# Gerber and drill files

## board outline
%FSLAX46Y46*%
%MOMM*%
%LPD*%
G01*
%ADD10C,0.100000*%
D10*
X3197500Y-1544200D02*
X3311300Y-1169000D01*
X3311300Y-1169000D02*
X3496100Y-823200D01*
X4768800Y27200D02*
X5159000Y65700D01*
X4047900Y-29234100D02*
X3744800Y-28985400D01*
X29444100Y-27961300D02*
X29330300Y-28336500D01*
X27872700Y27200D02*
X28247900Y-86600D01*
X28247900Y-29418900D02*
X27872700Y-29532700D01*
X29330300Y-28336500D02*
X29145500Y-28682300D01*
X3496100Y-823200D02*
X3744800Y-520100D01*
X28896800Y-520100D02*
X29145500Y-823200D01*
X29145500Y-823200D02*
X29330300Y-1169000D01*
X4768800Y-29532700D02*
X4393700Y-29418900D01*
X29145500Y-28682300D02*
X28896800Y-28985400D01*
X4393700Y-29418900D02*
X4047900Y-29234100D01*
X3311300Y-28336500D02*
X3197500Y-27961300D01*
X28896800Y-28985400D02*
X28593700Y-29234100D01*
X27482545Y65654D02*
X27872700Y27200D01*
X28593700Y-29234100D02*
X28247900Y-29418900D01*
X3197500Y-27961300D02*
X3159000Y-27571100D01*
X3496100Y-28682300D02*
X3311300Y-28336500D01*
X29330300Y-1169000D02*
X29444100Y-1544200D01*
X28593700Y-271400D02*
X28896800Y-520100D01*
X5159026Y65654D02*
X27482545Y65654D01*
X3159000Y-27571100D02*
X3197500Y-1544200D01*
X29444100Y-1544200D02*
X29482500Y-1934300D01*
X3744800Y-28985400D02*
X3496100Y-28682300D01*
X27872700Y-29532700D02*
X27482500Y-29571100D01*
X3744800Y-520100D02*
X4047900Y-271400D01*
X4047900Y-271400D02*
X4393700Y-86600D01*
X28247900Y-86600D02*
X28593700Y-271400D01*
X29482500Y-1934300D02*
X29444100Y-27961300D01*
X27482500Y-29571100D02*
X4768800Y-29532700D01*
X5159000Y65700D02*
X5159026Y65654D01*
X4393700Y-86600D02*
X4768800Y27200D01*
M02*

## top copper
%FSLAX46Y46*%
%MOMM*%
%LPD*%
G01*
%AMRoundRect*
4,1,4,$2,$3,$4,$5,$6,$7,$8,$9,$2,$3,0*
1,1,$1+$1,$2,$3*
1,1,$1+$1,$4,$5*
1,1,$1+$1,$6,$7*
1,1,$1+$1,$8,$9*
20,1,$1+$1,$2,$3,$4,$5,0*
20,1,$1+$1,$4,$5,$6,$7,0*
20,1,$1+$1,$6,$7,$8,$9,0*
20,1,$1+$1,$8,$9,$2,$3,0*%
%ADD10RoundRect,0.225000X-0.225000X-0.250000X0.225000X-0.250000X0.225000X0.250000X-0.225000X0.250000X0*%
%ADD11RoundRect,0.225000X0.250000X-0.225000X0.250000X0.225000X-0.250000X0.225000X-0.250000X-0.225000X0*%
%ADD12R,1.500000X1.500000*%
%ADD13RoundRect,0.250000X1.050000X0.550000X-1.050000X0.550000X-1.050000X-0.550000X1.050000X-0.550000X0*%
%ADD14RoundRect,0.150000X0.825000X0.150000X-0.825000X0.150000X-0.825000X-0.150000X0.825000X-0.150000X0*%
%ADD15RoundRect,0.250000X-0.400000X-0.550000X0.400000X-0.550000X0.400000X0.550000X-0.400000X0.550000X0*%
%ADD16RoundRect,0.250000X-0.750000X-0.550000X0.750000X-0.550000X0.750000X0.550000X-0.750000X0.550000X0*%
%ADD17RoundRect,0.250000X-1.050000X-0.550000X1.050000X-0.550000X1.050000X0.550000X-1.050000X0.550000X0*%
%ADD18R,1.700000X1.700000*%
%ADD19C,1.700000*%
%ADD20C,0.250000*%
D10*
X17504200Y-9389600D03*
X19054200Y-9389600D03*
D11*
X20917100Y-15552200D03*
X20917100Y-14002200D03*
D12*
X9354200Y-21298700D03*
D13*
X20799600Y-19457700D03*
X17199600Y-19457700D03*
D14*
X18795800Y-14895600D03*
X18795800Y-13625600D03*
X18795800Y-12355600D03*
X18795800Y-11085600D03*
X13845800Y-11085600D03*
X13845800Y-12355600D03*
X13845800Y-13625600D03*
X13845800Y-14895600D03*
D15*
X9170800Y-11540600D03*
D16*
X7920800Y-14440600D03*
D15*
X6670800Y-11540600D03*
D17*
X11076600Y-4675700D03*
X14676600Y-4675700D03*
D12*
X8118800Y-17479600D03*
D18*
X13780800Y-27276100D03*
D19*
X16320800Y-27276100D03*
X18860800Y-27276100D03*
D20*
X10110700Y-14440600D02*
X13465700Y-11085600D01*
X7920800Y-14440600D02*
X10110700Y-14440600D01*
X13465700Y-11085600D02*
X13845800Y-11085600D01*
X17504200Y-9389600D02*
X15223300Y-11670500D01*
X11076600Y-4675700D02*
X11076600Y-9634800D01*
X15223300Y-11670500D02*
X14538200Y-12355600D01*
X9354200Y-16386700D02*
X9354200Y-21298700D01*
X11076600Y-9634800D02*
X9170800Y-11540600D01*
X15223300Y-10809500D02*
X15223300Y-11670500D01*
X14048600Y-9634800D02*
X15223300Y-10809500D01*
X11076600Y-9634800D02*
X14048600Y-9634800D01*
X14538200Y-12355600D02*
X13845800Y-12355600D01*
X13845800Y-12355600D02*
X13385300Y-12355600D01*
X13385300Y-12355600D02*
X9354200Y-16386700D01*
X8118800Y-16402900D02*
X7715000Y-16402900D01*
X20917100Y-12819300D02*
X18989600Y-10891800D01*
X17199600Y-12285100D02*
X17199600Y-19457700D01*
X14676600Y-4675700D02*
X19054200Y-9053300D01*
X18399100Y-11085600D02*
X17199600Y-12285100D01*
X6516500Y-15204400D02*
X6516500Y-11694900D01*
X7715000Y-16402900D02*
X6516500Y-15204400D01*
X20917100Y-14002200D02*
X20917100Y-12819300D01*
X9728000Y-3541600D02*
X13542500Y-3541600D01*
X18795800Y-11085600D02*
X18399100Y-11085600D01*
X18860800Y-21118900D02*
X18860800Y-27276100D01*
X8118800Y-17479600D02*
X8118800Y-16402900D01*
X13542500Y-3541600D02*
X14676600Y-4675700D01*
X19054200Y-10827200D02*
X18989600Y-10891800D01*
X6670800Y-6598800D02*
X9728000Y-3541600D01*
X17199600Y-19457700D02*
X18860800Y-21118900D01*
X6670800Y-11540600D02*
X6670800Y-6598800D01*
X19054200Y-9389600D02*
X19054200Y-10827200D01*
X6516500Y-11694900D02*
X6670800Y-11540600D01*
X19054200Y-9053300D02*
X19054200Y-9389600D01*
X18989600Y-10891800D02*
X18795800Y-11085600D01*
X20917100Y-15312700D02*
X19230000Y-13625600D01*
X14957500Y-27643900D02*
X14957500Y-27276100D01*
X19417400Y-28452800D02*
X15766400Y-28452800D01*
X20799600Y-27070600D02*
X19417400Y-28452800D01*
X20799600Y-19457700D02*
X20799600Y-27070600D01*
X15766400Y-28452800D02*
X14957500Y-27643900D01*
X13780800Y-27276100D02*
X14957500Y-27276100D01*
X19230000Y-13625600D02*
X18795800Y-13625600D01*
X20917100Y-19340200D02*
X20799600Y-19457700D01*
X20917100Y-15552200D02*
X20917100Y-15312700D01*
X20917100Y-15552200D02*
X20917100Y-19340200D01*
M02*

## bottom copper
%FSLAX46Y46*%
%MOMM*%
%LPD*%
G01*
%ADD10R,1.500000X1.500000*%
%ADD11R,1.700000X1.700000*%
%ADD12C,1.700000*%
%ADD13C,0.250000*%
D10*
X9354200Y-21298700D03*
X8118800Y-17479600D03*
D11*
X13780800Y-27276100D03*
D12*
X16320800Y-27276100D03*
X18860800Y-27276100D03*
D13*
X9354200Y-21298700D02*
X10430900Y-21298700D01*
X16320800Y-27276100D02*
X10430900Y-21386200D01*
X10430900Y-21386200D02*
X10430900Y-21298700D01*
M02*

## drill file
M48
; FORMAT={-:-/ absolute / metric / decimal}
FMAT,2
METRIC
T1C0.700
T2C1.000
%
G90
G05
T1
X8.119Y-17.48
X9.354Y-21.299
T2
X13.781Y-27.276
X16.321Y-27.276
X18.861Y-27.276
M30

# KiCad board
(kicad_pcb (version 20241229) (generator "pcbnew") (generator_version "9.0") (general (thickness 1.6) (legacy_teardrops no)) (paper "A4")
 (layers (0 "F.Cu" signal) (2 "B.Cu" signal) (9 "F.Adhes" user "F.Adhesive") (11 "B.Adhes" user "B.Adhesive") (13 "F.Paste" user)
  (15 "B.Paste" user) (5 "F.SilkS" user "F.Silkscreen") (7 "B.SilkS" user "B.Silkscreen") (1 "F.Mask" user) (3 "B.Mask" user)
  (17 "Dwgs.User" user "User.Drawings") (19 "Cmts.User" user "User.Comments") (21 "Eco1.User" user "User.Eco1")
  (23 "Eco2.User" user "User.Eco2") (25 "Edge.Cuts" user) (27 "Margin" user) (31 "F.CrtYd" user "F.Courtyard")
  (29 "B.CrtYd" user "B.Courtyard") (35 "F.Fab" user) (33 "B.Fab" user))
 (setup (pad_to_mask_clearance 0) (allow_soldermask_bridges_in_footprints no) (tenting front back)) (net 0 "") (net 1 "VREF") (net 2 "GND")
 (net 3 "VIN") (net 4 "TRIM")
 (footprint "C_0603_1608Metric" (layer "F.Cu") (at 18.2792 9.3896)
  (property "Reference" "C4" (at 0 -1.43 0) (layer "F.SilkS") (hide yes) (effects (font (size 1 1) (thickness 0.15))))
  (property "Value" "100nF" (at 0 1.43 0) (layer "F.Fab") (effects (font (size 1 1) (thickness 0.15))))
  (pad "1" smd roundrect (at -0.775 0) (size 0.9 0.95) (layers "F.Cu" "F.Mask" "F.Paste") (roundrect_rratio 0.25) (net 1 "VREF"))
  (pad "2" smd roundrect (at 0.775 0) (size 0.9 0.95) (layers "F.Cu" "F.Mask" "F.Paste") (roundrect_rratio 0.25) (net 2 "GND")))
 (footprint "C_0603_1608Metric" (layer "F.Cu") (at 20.9171 14.7772 90)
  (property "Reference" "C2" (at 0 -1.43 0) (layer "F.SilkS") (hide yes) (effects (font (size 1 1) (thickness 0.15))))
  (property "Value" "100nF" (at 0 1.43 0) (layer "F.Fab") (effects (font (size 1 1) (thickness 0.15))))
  (pad "1" smd roundrect (at -0.775 0 90) (size 0.9 0.95) (layers "F.Cu" "F.Mask" "F.Paste") (roundrect_rratio 0.25) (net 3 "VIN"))
  (pad "2" smd roundrect (at 0.775 0 90) (size 0.9 0.95) (layers "F.Cu" "F.Mask" "F.Paste") (roundrect_rratio 0.25) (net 2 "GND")))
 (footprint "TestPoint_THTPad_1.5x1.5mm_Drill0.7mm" (layer "F.Cu") (at 9.3542 21.2987)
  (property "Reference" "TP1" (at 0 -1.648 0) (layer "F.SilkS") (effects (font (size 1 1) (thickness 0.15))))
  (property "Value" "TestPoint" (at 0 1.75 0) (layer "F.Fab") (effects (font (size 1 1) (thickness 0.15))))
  (pad "1" thru_hole rect (at 0 0) (size 1.5 1.5) (drill 0.7) (layers "*.Cu" "*.Mask") (remove_unused_layers no) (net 1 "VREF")))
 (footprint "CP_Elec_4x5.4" (layer "F.Cu") (at 18.9996 19.4577 180)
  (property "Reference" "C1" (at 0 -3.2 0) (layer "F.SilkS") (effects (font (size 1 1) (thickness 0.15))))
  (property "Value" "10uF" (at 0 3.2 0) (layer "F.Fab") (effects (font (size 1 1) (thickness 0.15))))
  (pad "1" smd roundrect (at -1.8 0 180) (size 2.6 1.6) (layers "F.Cu" "F.Mask" "F.Paste") (roundrect_rratio 0.15625) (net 3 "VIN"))
  (pad "2" smd roundrect (at 1.8 0 180) (size 2.6 1.6) (layers "F.Cu" "F.Mask" "F.Paste") (roundrect_rratio 0.15625) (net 2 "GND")))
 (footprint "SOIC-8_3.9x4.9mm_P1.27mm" (layer "F.Cu") (at 16.3208 12.9906 180)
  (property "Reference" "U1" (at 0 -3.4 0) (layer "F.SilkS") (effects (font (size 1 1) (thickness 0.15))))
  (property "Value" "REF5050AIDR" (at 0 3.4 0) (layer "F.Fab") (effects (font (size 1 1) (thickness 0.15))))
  (pad "1" smd roundrect (at -2.475 -1.905 180) (size 1.95 0.6) (layers "F.Cu" "F.Mask" "F.Paste") (roundrect_rratio 0.25))
  (pad "2" smd roundrect (at -2.475 -0.635 180) (size 1.95 0.6) (layers "F.Cu" "F.Mask" "F.Paste") (roundrect_rratio 0.25) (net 3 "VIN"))
  (pad "3" smd roundrect (at -2.475 0.635 180) (size 1.95 0.6) (layers "F.Cu" "F.Mask" "F.Paste") (roundrect_rratio 0.25))
  (pad "4" smd roundrect (at -2.475 1.905 180) (size 1.95 0.6) (layers "F.Cu" "F.Mask" "F.Paste") (roundrect_rratio 0.25) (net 2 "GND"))
  (pad "5" smd roundrect (at 2.475 1.905 180) (size 1.95 0.6) (layers "F.Cu" "F.Mask" "F.Paste") (roundrect_rratio 0.25) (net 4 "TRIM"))
  (pad "6" smd roundrect (at 2.475 0.635 180) (size 1.95 0.6) (layers "F.Cu" "F.Mask" "F.Paste") (roundrect_rratio 0.25) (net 1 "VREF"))
  (pad "7" smd roundrect (at 2.475 -0.635 180) (size 1.95 0.6) (layers "F.Cu" "F.Mask" "F.Paste") (roundrect_rratio 0.25))
  (pad "8" smd roundrect (at 2.475 -1.905 180) (size 1.95 0.6) (layers "F.Cu" "F.Mask" "F.Paste") (roundrect_rratio 0.25)))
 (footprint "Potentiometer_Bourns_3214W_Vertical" (layer "F.Cu") (at 7.9208 12.9906)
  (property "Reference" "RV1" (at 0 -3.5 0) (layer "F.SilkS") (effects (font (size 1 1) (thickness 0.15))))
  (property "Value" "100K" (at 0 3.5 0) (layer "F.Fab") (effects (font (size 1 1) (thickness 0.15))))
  (pad "1" smd roundrect (at 1.25 -1.45) (size 1.3 1.6) (layers "F.Cu" "F.Mask" "F.Paste") (roundrect_rratio 0.192308) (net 1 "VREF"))
  (pad "2" smd roundrect (at 0 1.45) (size 2 1.6) (layers "F.Cu" "F.Mask" "F.Paste") (roundrect_rratio 0.15625) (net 4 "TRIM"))
  (pad "3" smd roundrect (at -1.25 -1.45) (size 1.3 1.6) (layers "F.Cu" "F.Mask" "F.Paste") (roundrect_rratio 0.192308) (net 2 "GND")))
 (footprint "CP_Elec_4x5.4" (layer "F.Cu") (at 12.8766 4.6757)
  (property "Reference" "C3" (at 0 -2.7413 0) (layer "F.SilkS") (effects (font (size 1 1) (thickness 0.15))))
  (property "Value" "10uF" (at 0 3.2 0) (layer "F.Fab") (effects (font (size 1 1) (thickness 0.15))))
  (pad "1" smd roundrect (at -1.8 0) (size 2.6 1.6) (layers "F.Cu" "F.Mask" "F.Paste") (roundrect_rratio 0.15625) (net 1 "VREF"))
  (pad "2" smd roundrect (at 1.8 0) (size 2.6 1.6) (layers "F.Cu" "F.Mask" "F.Paste") (roundrect_rratio 0.15625) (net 2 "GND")))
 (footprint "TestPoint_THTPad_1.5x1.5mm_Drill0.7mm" (layer "F.Cu") (at 8.1188 17.4796)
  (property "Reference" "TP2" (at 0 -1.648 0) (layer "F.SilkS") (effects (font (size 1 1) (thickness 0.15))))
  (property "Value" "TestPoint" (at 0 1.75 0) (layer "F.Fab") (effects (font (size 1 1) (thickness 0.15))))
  (pad "1" thru_hole rect (at 0 0) (size 1.5 1.5) (drill 0.7) (layers "*.Cu" "*.Mask") (remove_unused_layers no) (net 2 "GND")))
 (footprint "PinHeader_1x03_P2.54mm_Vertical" (layer "F.Cu") (at 13.7808 27.2761 90)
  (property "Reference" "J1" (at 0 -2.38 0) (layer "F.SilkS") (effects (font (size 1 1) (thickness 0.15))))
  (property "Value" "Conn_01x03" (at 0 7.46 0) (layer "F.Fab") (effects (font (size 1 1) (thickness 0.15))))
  (pad "1" thru_hole rect (at 0 0 90) (size 1.7 1.7) (drill 1) (layers "*.Cu" "*.Mask") (remove_unused_layers no) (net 3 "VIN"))
  (pad "2" thru_hole circle (at 0 2.54 90) (size 1.7 1.7) (drill 1) (layers "*.Cu" "*.Mask") (remove_unused_layers no) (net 1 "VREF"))
  (pad "3" thru_hole circle (at 0 5.08 90) (size 1.7 1.7) (drill 1) (layers "*.Cu" "*.Mask") (remove_unused_layers no) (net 2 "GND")))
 (gr_line (start 3.1975 1.5442) (end 3.3113 1.169) (stroke (width 0.1) (type solid)) (layer "Edge.Cuts"))
 (gr_line (start 3.3113 1.169) (end 3.4961 0.8232) (stroke (width 0.1) (type solid)) (layer "Edge.Cuts"))
 (gr_line (start 4.7688 -0.0272) (end 5.159 -0.0657) (stroke (width 0.1) (type solid)) (layer "Edge.Cuts"))
 (gr_line (start 4.0479 29.2341) (end 3.7448 28.9854) (stroke (width 0.1) (type solid)) (layer "Edge.Cuts"))
 (gr_line (start 29.4441 27.9613) (end 29.3303 28.3365) (stroke (width 0.1) (type solid)) (layer "Edge.Cuts"))
 (gr_line (start 27.8727 -0.0272) (end 28.2479 0.0866) (stroke (width 0.1) (type solid)) (layer "Edge.Cuts"))
 (gr_line (start 28.2479 29.4189) (end 27.8727 29.5327) (stroke (width 0.1) (type solid)) (layer "Edge.Cuts"))
 (gr_line (start 29.3303 28.3365) (end 29.1455 28.6823) (stroke (width 0.1) (type solid)) (layer "Edge.Cuts"))
 (gr_line (start 3.4961 0.8232) (end 3.7448 0.5201) (stroke (width 0.1) (type solid)) (layer "Edge.Cuts"))
 (gr_line (start 28.8968 0.5201) (end 29.1455 0.8232) (stroke (width 0.1) (type solid)) (layer "Edge.Cuts"))
 (gr_line (start 29.1455 0.8232) (end 29.3303 1.169) (stroke (width 0.1) (type solid)) (layer "Edge.Cuts"))
 (gr_line (start 4.7688 29.5327) (end 4.3937 29.4189) (stroke (width 0.1) (type solid)) (layer "Edge.Cuts"))
 (gr_line (start 29.1455 28.6823) (end 28.8968 28.9854) (stroke (width 0.1) (type solid)) (layer "Edge.Cuts"))
 (gr_line (start 4.3937 29.4189) (end 4.0479 29.2341) (stroke (width 0.1) (type solid)) (layer "Edge.Cuts"))
 (gr_line (start 3.3113 28.3365) (end 3.1975 27.9613) (stroke (width 0.1) (type solid)) (layer "Edge.Cuts"))
 (gr_line (start 28.8968 28.9854) (end 28.5937 29.2341) (stroke (width 0.1) (type solid)) (layer "Edge.Cuts"))
 (gr_line (start 27.482545 -0.065654) (end 27.8727 -0.0272) (stroke (width 0.1) (type solid)) (layer "Edge.Cuts"))
 (gr_line (start 28.5937 29.2341) (end 28.2479 29.4189) (stroke (width 0.1) (type solid)) (layer "Edge.Cuts"))
 (gr_line (start 3.1975 27.9613) (end 3.159 27.5711) (stroke (width 0.1) (type solid)) (layer "Edge.Cuts"))
 (gr_line (start 3.4961 28.6823) (end 3.3113 28.3365) (stroke (width 0.1) (type solid)) (layer "Edge.Cuts"))
 (gr_line (start 29.3303 1.169) (end 29.4441 1.5442) (stroke (width 0.1) (type solid)) (layer "Edge.Cuts"))
 (gr_line (start 28.5937 0.2714) (end 28.8968 0.5201) (stroke (width 0.1) (type solid)) (layer "Edge.Cuts"))
 (gr_line (start 5.159026 -0.065654) (end 27.482545 -0.065654) (stroke (width 0.1) (type solid)) (layer "Edge.Cuts"))
 (gr_line (start 3.159 27.5711) (end 3.1975 1.5442) (stroke (width 0.1) (type solid)) (layer "Edge.Cuts"))
 (gr_line (start 29.4441 1.5442) (end 29.4825 1.9343) (stroke (width 0.1) (type solid)) (layer "Edge.Cuts"))
 (gr_line (start 3.7448 28.9854) (end 3.4961 28.6823) (stroke (width 0.1) (type solid)) (layer "Edge.Cuts"))
 (gr_line (start 27.8727 29.5327) (end 27.4825 29.5711) (stroke (width 0.1) (type solid)) (layer "Edge.Cuts"))
 (gr_line (start 3.7448 0.5201) (end 4.0479 0.2714) (stroke (width 0.1) (type solid)) (layer "Edge.Cuts"))
 (gr_line (start 4.0479 0.2714) (end 4.3937 0.0866) (stroke (width 0.1) (type solid)) (layer "Edge.Cuts"))
 (gr_line (start 28.2479 0.0866) (end 28.5937 0.2714) (stroke (width 0.1) (type solid)) (layer "Edge.Cuts"))
 (gr_line (start 29.4825 1.9343) (end 29.4441 27.9613) (stroke (width 0.1) (type solid)) (layer "Edge.Cuts"))
 (gr_line (start 27.4825 29.5711) (end 4.7688 29.5327) (stroke (width 0.1) (type solid)) (layer "Edge.Cuts"))
 (gr_line (start 5.159 -0.0657) (end 5.159026 -0.065654) (stroke (width 0.1) (type solid)) (layer "Edge.Cuts"))
 (gr_line (start 4.3937 0.0866) (end 4.7688 -0.0272) (stroke (width 0.1) (type solid)) (layer "Edge.Cuts"))
 (segment (start 10.1107 14.4406) (end 13.4657 11.0856) (width 0.25) (layer "F.Cu") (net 4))
 (segment (start 7.9208 14.4406) (end 10.1107 14.4406) (width 0.25) (layer "F.Cu") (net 4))
 (segment (start 13.4657 11.0856) (end 13.8458 11.0856) (width 0.25) (layer "F.Cu") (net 4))
 (segment (start 17.5042 9.3896) (end 15.2233 11.6705) (width 0.25) (layer "F.Cu") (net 1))
 (segment (start 11.0766 4.6757) (end 11.0766 9.6348) (width 0.25) (layer "F.Cu") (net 1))
 (segment (start 15.2233 11.6705) (end 14.5382 12.3556) (width 0.25) (layer "F.Cu") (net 1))
 (segment (start 9.3542 16.3867) (end 9.3542 21.2987) (width 0.25) (layer "F.Cu") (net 1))
 (segment (start 11.0766 9.6348) (end 9.1708 11.5406) (width 0.25) (layer "F.Cu") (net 1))
 (segment (start 15.2233 10.8095) (end 15.2233 11.6705) (width 0.25) (layer "F.Cu") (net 1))
 (segment (start 14.0486 9.6348) (end 15.2233 10.8095) (width 0.25) (layer "F.Cu") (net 1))
 (segment (start 11.0766 9.6348) (end 14.0486 9.6348) (width 0.25) (layer "F.Cu") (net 1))
 (segment (start 14.5382 12.3556) (end 13.8458 12.3556) (width 0.25) (layer "F.Cu") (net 1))
 (segment (start 13.8458 12.3556) (end 13.3853 12.3556) (width 0.25) (layer "F.Cu") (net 1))
 (segment (start 13.3853 12.3556) (end 9.3542 16.3867) (width 0.25) (layer "F.Cu") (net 1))
 (segment (start 9.3542 21.2987) (end 10.4309 21.2987) (width 0.25) (layer "B.Cu") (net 1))
 (segment (start 16.3208 27.2761) (end 10.4309 21.3862) (width 0.25) (layer "B.Cu") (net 1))
 (segment (start 10.4309 21.3862) (end 10.4309 21.2987) (width 0.25) (layer "B.Cu") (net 1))
 (segment (start 8.1188 16.4029) (end 7.715 16.4029) (width 0.25) (layer "F.Cu") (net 2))
 (segment (start 20.9171 12.8193) (end 18.9896 10.8918) (width 0.25) (layer "F.Cu") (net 2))
 (segment (start 17.1996 12.2851) (end 17.1996 19.4577) (width 0.25) (layer "F.Cu") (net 2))
 (segment (start 14.6766 4.6757) (end 19.0542 9.0533) (width 0.25) (layer "F.Cu") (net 2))
 (segment (start 18.3991 11.0856) (end 17.1996 12.2851) (width 0.25) (layer "F.Cu") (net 2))
 (segment (start 6.5165 15.2044) (end 6.5165 11.6949) (width 0.25) (layer "F.Cu") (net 2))
 (segment (start 7.715 16.4029) (end 6.5165 15.2044) (width 0.25) (layer "F.Cu") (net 2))
 (segment (start 20.9171 14.0022) (end 20.9171 12.8193) (width 0.25) (layer "F.Cu") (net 2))
 (segment (start 9.728 3.5416) (end 13.5425 3.5416) (width 0.25) (layer "F.Cu") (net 2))
 (segment (start 18.7958 11.0856) (end 18.3991 11.0856) (width 0.25) (layer "F.Cu") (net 2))
 (segment (start 18.8608 21.1189) (end 18.8608 27.2761) (width 0.25) (layer "F.Cu") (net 2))
 (segment (start 8.1188 17.4796) (end 8.1188 16.4029) (width 0.25) (layer "F.Cu") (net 2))
 (segment (start 13.5425 3.5416) (end 14.6766 4.6757) (width 0.25) (layer "F.Cu") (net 2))
 (segment (start 19.0542 10.8272) (end 18.9896 10.8918) (width 0.25) (layer "F.Cu") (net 2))
 (segment (start 6.6708 6.5988) (end 9.728 3.5416) (width 0.25) (layer "F.Cu") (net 2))
 (segment (start 17.1996 19.4577) (end 18.8608 21.1189) (width 0.25) (layer "F.Cu") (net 2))
 (segment (start 6.6708 11.5406) (end 6.6708 6.5988) (width 0.25) (layer "F.Cu") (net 2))
 (segment (start 19.0542 9.3896) (end 19.0542 10.8272) (width 0.25) (layer "F.Cu") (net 2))
 (segment (start 6.5165 11.6949) (end 6.6708 11.5406) (width 0.25) (layer "F.Cu") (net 2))
 (segment (start 19.0542 9.0533) (end 19.0542 9.3896) (width 0.25) (layer "F.Cu") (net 2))
 (segment (start 18.9896 10.8918) (end 18.7958 11.0856) (width 0.25) (layer "F.Cu") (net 2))
 (segment (start 20.9171 15.3127) (end 19.23 13.6256) (width 0.25) (layer "F.Cu") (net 3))
 (segment (start 14.9575 27.6439) (end 14.9575 27.2761) (width 0.25) (layer "F.Cu") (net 3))
 (segment (start 19.4174 28.4528) (end 15.7664 28.4528) (width 0.25) (layer "F.Cu") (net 3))
 (segment (start 20.7996 27.0706) (end 19.4174 28.4528) (width 0.25) (layer "F.Cu") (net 3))
 (segment (start 20.7996 19.4577) (end 20.7996 27.0706) (width 0.25) (layer "F.Cu") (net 3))
 (segment (start 15.7664 28.4528) (end 14.9575 27.6439) (width 0.25) (layer "F.Cu") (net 3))
 (segment (start 13.7808 27.2761) (end 14.9575 27.2761) (width 0.25) (layer "F.Cu") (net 3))
 (segment (start 19.23 13.6256) (end 18.7958 13.6256) (width 0.25) (layer "F.Cu") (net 3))
 (segment (start 20.9171 19.3402) (end 20.7996 19.4577) (width 0.25) (layer "F.Cu") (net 3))
 (segment (start 20.9171 15.5522) (end 20.9171 15.3127) (width 0.25) (layer "F.Cu") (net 3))
 (segment (start 20.9171 15.5522) (end 20.9171 19.3402) (width 0.25) (layer "F.Cu") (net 3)))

